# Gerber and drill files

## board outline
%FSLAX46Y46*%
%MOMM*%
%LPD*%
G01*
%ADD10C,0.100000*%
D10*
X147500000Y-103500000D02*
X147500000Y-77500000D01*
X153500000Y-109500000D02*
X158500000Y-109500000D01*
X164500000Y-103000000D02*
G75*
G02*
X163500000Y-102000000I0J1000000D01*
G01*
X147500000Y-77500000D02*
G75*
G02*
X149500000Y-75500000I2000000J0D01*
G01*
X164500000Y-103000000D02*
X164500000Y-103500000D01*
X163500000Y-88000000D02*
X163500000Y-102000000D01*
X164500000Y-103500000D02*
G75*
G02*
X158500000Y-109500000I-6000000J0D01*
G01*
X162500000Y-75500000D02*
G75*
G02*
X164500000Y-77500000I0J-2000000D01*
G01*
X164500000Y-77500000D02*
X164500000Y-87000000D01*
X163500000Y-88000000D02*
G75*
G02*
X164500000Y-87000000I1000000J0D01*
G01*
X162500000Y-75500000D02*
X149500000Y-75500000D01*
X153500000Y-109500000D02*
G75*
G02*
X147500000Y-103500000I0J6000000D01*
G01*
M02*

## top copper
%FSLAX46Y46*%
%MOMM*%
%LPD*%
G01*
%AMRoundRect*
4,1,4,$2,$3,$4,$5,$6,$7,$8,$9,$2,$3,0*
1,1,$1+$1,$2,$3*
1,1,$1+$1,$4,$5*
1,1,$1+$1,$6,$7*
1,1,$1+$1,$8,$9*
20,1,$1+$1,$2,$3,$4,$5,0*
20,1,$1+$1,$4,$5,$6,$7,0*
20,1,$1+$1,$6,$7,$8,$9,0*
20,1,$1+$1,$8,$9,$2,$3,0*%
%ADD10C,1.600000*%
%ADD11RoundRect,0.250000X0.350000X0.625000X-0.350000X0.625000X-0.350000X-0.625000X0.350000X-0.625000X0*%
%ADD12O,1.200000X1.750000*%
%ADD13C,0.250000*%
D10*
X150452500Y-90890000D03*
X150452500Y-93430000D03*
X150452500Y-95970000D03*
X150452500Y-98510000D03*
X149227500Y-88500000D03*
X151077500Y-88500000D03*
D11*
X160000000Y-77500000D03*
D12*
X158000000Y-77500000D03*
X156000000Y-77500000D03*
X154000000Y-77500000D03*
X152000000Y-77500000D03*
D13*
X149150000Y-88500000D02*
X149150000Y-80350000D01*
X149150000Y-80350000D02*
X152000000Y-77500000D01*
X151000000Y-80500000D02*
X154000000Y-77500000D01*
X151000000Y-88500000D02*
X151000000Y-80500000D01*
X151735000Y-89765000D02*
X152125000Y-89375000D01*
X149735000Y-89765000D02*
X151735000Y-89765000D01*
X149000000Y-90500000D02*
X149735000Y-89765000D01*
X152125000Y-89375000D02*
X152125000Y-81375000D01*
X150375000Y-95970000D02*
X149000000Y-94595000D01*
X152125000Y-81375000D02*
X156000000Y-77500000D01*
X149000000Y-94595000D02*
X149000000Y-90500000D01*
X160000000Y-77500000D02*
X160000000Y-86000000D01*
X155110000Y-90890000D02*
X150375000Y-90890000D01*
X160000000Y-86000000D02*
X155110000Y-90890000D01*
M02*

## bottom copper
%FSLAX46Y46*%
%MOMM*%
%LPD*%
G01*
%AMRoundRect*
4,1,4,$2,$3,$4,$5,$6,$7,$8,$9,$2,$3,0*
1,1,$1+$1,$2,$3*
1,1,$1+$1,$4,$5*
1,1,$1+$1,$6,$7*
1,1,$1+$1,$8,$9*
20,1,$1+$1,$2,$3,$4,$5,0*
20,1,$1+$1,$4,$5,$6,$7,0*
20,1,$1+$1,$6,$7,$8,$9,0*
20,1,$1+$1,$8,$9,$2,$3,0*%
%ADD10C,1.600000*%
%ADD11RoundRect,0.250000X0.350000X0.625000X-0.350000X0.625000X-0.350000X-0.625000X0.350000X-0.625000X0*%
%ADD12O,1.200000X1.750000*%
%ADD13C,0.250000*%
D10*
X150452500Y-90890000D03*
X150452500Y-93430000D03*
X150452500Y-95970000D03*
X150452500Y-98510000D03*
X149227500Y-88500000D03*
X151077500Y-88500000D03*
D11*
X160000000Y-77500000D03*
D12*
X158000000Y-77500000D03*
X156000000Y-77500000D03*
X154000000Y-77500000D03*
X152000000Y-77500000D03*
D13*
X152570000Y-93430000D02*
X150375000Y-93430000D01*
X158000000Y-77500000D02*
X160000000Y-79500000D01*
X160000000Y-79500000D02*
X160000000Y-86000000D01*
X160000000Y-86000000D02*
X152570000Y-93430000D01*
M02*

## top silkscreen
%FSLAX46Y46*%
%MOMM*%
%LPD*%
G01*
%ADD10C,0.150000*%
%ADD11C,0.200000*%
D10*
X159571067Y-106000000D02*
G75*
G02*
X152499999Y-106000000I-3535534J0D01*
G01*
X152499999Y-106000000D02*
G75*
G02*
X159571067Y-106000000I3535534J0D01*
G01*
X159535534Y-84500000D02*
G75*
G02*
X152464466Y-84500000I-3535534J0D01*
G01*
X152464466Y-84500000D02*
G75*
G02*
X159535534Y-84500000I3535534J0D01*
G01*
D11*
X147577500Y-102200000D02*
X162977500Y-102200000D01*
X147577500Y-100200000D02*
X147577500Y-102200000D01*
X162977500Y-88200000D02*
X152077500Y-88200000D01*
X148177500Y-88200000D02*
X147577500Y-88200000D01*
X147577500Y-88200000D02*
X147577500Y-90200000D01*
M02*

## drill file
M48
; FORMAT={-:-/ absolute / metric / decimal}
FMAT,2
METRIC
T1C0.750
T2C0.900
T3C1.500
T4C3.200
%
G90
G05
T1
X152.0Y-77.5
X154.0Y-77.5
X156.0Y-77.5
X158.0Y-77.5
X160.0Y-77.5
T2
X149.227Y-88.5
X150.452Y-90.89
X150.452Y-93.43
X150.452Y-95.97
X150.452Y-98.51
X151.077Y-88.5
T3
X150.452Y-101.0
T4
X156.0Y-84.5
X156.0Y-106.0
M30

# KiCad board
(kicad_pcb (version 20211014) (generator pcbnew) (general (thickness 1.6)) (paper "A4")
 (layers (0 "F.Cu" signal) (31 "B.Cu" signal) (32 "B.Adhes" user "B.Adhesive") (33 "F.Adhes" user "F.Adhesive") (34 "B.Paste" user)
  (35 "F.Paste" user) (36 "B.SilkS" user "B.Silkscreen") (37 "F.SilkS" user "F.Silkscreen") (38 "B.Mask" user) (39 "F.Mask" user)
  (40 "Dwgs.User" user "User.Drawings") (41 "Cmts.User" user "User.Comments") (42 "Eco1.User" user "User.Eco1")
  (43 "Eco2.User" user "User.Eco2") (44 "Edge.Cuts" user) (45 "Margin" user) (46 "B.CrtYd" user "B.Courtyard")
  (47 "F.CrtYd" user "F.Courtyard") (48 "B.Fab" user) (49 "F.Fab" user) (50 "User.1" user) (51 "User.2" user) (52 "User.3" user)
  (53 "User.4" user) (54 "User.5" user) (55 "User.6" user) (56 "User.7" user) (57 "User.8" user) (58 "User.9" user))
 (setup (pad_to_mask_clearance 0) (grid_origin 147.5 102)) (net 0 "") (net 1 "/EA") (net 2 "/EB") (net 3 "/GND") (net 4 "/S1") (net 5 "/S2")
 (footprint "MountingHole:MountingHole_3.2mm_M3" (layer "F.Cu") (at 156 84.5)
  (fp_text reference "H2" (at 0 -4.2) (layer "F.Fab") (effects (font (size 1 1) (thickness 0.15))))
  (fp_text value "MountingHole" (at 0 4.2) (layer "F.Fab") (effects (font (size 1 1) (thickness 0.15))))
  (pad "" np_thru_hole circle (at 0 0) (size 3.2 3.2) (drill 3.2) (layers *.Cu *.Mask)))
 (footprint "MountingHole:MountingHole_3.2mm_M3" (layer "F.Cu") (at 156 106)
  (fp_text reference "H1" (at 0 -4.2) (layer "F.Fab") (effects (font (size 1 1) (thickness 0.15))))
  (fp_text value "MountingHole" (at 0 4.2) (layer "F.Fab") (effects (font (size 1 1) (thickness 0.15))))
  (pad "" np_thru_hole circle (at 0 0) (size 3.2 3.2) (drill 3.2) (layers *.Cu *.Mask)))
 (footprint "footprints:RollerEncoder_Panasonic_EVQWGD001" (layer "F.Cu") (at 156.0775 94.7)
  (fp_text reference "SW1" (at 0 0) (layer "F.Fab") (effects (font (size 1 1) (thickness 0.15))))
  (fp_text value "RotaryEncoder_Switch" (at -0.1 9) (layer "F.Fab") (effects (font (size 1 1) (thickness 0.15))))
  (fp_line (start -8.5 7.5) (end 6.9 7.5) (layer "F.SilkS") (width 0.2))
  (fp_line (start -8.5 5.5) (end -8.5 7.5) (layer "F.SilkS") (width 0.2))
  (fp_line (start 6.9 -6.5) (end -4 -6.5) (layer "F.SilkS") (width 0.2))
  (fp_line (start -7.9 -6.5) (end -8.5 -6.5) (layer "F.SilkS") (width 0.2))
  (fp_line (start -8.5 -6.5) (end -8.5 -4.5) (layer "F.SilkS") (width 0.2))
  (pad "" np_thru_hole circle (at -5.625 6.3) (size 1.5 1.5) (drill 1.5) (layers *.Cu *.Mask))
  (pad "A" thru_hole circle (at -5.625 -3.81) (size 1.6 1.6) (drill 0.9) (layers *.Cu *.Mask) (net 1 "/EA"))
  (pad "B" thru_hole circle (at -5.625 -1.27) (size 1.6 1.6) (drill 0.9) (layers *.Cu *.Mask) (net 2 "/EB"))
  (pad "C" thru_hole circle (at -5.625 1.27) (size 1.6 1.6) (drill 0.9) (layers *.Cu *.Mask) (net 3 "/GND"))
  (pad "NC" thru_hole circle (at -5.625 3.81) (size 1.6 1.6) (drill 0.9) (layers *.Cu *.Mask))
  (pad "S1" thru_hole circle (at -6.85 -6.2) (size 1.6 1.6) (drill 0.9) (layers *.Cu *.Mask) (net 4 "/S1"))
  (pad "S2" thru_hole circle (at -5 -6.2) (size 1.6 1.6) (drill 0.9) (layers *.Cu *.Mask) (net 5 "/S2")))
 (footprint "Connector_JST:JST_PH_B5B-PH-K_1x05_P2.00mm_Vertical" (layer "B.Cu") (at 160 77.5 180)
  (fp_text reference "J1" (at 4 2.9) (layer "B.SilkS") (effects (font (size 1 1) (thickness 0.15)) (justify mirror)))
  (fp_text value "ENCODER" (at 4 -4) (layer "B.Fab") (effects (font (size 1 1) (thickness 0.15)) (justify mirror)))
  (pad "1" thru_hole roundrect (at 0 0 180) (size 1.2 1.75) (drill 0.75) (layers *.Cu *.Mask) (roundrect_rratio 0.208333) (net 1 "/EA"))
  (pad "2" thru_hole oval (at 2 0 180) (size 1.2 1.75) (drill 0.75) (layers *.Cu *.Mask) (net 2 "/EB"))
  (pad "3" thru_hole oval (at 4 0 180) (size 1.2 1.75) (drill 0.75) (layers *.Cu *.Mask) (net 3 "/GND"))
  (pad "4" thru_hole oval (at 6 0 180) (size 1.2 1.75) (drill 0.75) (layers *.Cu *.Mask) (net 5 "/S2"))
  (pad "5" thru_hole oval (at 8 0 180) (size 1.2 1.75) (drill 0.75) (layers *.Cu *.Mask) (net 4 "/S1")))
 (gr_circle (center 156.035533 106) (end 159.535533 105.5) (layer "F.SilkS") (width 0.15) (fill none))
 (gr_circle (center 156 84.5) (end 159.5 84) (layer "F.SilkS") (width 0.15) (fill none))
 (gr_line (start 147.5 103.5) (end 147.5 77.5) (layer "Edge.Cuts") (width 0.1))
 (gr_line (start 153.5 109.5) (end 158.5 109.5) (layer "Edge.Cuts") (width 0.1))
 (gr_arc (start 164.5 103) (mid 163.792893 102.707107) (end 163.5 102) (layer "Edge.Cuts") (width 0.1))
 (gr_arc (start 147.5 77.5) (mid 148.085786 76.085786) (end 149.5 75.5) (layer "Edge.Cuts") (width 0.1))
 (gr_line (start 164.5 103) (end 164.5 103.5) (layer "Edge.Cuts") (width 0.1))
 (gr_line (start 163.5 88) (end 163.5 102) (layer "Edge.Cuts") (width 0.1))
 (gr_arc (start 164.5 103.5) (mid 162.742641 107.742641) (end 158.5 109.5) (layer "Edge.Cuts") (width 0.1))
 (gr_arc (start 162.5 75.5) (mid 163.914214 76.085786) (end 164.5 77.5) (layer "Edge.Cuts") (width 0.1))
 (gr_line (start 164.5 77.5) (end 164.5 87) (layer "Edge.Cuts") (width 0.1))
 (gr_arc (start 163.5 88) (mid 163.792893 87.292893) (end 164.5 87) (layer "Edge.Cuts") (width 0.1))
 (gr_line (start 162.5 75.5) (end 149.5 75.5) (layer "Edge.Cuts") (width 0.1))
 (gr_arc (start 153.5 109.5) (mid 149.257359 107.742641) (end 147.5 103.5) (layer "Edge.Cuts") (width 0.1))
 (segment (start 149.15 88.5) (end 149.15 80.35) (width 0.25) (layer "F.Cu") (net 4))
 (segment (start 149.15 80.35) (end 152 77.5) (width 0.25) (layer "F.Cu") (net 4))
 (segment (start 151 80.5) (end 154 77.5) (width 0.25) (layer "F.Cu") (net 5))
 (segment (start 151 88.5) (end 151 80.5) (width 0.25) (layer "F.Cu") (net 5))
 (segment (start 151.735 89.765) (end 152.125 89.375) (width 0.25) (layer "F.Cu") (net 3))
 (segment (start 149.735 89.765) (end 151.735 89.765) (width 0.25) (layer "F.Cu") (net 3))
 (segment (start 149 90.5) (end 149.735 89.765) (width 0.25) (layer "F.Cu") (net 3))
 (segment (start 152.125 89.375) (end 152.125 81.375) (width 0.25) (layer "F.Cu") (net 3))
 (segment (start 150.375 95.97) (end 149 94.595) (width 0.25) (layer "F.Cu") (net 3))
 (segment (start 152.125 81.375) (end 156 77.5) (width 0.25) (layer "F.Cu") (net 3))
 (segment (start 149 94.595) (end 149 90.5) (width 0.25) (layer "F.Cu") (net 3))
 (segment (start 160 77.5) (end 160 86) (width 0.25) (layer "F.Cu") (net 1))
 (segment (start 155.11 90.89) (end 150.375 90.89) (width 0.25) (layer "F.Cu") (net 1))
 (segment (start 160 86) (end 155.11 90.89) (width 0.25) (layer "F.Cu") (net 1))
 (segment (start 152.57 93.43) (end 150.375 93.43) (width 0.25) (layer "B.Cu") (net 2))
 (segment (start 158 77.5) (end 160 79.5) (width 0.25) (layer "B.Cu") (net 2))
 (segment (start 160 79.5) (end 160 86) (width 0.25) (layer "B.Cu") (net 2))
 (segment (start 160 86) (end 152.57 93.43) (width 0.25) (layer "B.Cu") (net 2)))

